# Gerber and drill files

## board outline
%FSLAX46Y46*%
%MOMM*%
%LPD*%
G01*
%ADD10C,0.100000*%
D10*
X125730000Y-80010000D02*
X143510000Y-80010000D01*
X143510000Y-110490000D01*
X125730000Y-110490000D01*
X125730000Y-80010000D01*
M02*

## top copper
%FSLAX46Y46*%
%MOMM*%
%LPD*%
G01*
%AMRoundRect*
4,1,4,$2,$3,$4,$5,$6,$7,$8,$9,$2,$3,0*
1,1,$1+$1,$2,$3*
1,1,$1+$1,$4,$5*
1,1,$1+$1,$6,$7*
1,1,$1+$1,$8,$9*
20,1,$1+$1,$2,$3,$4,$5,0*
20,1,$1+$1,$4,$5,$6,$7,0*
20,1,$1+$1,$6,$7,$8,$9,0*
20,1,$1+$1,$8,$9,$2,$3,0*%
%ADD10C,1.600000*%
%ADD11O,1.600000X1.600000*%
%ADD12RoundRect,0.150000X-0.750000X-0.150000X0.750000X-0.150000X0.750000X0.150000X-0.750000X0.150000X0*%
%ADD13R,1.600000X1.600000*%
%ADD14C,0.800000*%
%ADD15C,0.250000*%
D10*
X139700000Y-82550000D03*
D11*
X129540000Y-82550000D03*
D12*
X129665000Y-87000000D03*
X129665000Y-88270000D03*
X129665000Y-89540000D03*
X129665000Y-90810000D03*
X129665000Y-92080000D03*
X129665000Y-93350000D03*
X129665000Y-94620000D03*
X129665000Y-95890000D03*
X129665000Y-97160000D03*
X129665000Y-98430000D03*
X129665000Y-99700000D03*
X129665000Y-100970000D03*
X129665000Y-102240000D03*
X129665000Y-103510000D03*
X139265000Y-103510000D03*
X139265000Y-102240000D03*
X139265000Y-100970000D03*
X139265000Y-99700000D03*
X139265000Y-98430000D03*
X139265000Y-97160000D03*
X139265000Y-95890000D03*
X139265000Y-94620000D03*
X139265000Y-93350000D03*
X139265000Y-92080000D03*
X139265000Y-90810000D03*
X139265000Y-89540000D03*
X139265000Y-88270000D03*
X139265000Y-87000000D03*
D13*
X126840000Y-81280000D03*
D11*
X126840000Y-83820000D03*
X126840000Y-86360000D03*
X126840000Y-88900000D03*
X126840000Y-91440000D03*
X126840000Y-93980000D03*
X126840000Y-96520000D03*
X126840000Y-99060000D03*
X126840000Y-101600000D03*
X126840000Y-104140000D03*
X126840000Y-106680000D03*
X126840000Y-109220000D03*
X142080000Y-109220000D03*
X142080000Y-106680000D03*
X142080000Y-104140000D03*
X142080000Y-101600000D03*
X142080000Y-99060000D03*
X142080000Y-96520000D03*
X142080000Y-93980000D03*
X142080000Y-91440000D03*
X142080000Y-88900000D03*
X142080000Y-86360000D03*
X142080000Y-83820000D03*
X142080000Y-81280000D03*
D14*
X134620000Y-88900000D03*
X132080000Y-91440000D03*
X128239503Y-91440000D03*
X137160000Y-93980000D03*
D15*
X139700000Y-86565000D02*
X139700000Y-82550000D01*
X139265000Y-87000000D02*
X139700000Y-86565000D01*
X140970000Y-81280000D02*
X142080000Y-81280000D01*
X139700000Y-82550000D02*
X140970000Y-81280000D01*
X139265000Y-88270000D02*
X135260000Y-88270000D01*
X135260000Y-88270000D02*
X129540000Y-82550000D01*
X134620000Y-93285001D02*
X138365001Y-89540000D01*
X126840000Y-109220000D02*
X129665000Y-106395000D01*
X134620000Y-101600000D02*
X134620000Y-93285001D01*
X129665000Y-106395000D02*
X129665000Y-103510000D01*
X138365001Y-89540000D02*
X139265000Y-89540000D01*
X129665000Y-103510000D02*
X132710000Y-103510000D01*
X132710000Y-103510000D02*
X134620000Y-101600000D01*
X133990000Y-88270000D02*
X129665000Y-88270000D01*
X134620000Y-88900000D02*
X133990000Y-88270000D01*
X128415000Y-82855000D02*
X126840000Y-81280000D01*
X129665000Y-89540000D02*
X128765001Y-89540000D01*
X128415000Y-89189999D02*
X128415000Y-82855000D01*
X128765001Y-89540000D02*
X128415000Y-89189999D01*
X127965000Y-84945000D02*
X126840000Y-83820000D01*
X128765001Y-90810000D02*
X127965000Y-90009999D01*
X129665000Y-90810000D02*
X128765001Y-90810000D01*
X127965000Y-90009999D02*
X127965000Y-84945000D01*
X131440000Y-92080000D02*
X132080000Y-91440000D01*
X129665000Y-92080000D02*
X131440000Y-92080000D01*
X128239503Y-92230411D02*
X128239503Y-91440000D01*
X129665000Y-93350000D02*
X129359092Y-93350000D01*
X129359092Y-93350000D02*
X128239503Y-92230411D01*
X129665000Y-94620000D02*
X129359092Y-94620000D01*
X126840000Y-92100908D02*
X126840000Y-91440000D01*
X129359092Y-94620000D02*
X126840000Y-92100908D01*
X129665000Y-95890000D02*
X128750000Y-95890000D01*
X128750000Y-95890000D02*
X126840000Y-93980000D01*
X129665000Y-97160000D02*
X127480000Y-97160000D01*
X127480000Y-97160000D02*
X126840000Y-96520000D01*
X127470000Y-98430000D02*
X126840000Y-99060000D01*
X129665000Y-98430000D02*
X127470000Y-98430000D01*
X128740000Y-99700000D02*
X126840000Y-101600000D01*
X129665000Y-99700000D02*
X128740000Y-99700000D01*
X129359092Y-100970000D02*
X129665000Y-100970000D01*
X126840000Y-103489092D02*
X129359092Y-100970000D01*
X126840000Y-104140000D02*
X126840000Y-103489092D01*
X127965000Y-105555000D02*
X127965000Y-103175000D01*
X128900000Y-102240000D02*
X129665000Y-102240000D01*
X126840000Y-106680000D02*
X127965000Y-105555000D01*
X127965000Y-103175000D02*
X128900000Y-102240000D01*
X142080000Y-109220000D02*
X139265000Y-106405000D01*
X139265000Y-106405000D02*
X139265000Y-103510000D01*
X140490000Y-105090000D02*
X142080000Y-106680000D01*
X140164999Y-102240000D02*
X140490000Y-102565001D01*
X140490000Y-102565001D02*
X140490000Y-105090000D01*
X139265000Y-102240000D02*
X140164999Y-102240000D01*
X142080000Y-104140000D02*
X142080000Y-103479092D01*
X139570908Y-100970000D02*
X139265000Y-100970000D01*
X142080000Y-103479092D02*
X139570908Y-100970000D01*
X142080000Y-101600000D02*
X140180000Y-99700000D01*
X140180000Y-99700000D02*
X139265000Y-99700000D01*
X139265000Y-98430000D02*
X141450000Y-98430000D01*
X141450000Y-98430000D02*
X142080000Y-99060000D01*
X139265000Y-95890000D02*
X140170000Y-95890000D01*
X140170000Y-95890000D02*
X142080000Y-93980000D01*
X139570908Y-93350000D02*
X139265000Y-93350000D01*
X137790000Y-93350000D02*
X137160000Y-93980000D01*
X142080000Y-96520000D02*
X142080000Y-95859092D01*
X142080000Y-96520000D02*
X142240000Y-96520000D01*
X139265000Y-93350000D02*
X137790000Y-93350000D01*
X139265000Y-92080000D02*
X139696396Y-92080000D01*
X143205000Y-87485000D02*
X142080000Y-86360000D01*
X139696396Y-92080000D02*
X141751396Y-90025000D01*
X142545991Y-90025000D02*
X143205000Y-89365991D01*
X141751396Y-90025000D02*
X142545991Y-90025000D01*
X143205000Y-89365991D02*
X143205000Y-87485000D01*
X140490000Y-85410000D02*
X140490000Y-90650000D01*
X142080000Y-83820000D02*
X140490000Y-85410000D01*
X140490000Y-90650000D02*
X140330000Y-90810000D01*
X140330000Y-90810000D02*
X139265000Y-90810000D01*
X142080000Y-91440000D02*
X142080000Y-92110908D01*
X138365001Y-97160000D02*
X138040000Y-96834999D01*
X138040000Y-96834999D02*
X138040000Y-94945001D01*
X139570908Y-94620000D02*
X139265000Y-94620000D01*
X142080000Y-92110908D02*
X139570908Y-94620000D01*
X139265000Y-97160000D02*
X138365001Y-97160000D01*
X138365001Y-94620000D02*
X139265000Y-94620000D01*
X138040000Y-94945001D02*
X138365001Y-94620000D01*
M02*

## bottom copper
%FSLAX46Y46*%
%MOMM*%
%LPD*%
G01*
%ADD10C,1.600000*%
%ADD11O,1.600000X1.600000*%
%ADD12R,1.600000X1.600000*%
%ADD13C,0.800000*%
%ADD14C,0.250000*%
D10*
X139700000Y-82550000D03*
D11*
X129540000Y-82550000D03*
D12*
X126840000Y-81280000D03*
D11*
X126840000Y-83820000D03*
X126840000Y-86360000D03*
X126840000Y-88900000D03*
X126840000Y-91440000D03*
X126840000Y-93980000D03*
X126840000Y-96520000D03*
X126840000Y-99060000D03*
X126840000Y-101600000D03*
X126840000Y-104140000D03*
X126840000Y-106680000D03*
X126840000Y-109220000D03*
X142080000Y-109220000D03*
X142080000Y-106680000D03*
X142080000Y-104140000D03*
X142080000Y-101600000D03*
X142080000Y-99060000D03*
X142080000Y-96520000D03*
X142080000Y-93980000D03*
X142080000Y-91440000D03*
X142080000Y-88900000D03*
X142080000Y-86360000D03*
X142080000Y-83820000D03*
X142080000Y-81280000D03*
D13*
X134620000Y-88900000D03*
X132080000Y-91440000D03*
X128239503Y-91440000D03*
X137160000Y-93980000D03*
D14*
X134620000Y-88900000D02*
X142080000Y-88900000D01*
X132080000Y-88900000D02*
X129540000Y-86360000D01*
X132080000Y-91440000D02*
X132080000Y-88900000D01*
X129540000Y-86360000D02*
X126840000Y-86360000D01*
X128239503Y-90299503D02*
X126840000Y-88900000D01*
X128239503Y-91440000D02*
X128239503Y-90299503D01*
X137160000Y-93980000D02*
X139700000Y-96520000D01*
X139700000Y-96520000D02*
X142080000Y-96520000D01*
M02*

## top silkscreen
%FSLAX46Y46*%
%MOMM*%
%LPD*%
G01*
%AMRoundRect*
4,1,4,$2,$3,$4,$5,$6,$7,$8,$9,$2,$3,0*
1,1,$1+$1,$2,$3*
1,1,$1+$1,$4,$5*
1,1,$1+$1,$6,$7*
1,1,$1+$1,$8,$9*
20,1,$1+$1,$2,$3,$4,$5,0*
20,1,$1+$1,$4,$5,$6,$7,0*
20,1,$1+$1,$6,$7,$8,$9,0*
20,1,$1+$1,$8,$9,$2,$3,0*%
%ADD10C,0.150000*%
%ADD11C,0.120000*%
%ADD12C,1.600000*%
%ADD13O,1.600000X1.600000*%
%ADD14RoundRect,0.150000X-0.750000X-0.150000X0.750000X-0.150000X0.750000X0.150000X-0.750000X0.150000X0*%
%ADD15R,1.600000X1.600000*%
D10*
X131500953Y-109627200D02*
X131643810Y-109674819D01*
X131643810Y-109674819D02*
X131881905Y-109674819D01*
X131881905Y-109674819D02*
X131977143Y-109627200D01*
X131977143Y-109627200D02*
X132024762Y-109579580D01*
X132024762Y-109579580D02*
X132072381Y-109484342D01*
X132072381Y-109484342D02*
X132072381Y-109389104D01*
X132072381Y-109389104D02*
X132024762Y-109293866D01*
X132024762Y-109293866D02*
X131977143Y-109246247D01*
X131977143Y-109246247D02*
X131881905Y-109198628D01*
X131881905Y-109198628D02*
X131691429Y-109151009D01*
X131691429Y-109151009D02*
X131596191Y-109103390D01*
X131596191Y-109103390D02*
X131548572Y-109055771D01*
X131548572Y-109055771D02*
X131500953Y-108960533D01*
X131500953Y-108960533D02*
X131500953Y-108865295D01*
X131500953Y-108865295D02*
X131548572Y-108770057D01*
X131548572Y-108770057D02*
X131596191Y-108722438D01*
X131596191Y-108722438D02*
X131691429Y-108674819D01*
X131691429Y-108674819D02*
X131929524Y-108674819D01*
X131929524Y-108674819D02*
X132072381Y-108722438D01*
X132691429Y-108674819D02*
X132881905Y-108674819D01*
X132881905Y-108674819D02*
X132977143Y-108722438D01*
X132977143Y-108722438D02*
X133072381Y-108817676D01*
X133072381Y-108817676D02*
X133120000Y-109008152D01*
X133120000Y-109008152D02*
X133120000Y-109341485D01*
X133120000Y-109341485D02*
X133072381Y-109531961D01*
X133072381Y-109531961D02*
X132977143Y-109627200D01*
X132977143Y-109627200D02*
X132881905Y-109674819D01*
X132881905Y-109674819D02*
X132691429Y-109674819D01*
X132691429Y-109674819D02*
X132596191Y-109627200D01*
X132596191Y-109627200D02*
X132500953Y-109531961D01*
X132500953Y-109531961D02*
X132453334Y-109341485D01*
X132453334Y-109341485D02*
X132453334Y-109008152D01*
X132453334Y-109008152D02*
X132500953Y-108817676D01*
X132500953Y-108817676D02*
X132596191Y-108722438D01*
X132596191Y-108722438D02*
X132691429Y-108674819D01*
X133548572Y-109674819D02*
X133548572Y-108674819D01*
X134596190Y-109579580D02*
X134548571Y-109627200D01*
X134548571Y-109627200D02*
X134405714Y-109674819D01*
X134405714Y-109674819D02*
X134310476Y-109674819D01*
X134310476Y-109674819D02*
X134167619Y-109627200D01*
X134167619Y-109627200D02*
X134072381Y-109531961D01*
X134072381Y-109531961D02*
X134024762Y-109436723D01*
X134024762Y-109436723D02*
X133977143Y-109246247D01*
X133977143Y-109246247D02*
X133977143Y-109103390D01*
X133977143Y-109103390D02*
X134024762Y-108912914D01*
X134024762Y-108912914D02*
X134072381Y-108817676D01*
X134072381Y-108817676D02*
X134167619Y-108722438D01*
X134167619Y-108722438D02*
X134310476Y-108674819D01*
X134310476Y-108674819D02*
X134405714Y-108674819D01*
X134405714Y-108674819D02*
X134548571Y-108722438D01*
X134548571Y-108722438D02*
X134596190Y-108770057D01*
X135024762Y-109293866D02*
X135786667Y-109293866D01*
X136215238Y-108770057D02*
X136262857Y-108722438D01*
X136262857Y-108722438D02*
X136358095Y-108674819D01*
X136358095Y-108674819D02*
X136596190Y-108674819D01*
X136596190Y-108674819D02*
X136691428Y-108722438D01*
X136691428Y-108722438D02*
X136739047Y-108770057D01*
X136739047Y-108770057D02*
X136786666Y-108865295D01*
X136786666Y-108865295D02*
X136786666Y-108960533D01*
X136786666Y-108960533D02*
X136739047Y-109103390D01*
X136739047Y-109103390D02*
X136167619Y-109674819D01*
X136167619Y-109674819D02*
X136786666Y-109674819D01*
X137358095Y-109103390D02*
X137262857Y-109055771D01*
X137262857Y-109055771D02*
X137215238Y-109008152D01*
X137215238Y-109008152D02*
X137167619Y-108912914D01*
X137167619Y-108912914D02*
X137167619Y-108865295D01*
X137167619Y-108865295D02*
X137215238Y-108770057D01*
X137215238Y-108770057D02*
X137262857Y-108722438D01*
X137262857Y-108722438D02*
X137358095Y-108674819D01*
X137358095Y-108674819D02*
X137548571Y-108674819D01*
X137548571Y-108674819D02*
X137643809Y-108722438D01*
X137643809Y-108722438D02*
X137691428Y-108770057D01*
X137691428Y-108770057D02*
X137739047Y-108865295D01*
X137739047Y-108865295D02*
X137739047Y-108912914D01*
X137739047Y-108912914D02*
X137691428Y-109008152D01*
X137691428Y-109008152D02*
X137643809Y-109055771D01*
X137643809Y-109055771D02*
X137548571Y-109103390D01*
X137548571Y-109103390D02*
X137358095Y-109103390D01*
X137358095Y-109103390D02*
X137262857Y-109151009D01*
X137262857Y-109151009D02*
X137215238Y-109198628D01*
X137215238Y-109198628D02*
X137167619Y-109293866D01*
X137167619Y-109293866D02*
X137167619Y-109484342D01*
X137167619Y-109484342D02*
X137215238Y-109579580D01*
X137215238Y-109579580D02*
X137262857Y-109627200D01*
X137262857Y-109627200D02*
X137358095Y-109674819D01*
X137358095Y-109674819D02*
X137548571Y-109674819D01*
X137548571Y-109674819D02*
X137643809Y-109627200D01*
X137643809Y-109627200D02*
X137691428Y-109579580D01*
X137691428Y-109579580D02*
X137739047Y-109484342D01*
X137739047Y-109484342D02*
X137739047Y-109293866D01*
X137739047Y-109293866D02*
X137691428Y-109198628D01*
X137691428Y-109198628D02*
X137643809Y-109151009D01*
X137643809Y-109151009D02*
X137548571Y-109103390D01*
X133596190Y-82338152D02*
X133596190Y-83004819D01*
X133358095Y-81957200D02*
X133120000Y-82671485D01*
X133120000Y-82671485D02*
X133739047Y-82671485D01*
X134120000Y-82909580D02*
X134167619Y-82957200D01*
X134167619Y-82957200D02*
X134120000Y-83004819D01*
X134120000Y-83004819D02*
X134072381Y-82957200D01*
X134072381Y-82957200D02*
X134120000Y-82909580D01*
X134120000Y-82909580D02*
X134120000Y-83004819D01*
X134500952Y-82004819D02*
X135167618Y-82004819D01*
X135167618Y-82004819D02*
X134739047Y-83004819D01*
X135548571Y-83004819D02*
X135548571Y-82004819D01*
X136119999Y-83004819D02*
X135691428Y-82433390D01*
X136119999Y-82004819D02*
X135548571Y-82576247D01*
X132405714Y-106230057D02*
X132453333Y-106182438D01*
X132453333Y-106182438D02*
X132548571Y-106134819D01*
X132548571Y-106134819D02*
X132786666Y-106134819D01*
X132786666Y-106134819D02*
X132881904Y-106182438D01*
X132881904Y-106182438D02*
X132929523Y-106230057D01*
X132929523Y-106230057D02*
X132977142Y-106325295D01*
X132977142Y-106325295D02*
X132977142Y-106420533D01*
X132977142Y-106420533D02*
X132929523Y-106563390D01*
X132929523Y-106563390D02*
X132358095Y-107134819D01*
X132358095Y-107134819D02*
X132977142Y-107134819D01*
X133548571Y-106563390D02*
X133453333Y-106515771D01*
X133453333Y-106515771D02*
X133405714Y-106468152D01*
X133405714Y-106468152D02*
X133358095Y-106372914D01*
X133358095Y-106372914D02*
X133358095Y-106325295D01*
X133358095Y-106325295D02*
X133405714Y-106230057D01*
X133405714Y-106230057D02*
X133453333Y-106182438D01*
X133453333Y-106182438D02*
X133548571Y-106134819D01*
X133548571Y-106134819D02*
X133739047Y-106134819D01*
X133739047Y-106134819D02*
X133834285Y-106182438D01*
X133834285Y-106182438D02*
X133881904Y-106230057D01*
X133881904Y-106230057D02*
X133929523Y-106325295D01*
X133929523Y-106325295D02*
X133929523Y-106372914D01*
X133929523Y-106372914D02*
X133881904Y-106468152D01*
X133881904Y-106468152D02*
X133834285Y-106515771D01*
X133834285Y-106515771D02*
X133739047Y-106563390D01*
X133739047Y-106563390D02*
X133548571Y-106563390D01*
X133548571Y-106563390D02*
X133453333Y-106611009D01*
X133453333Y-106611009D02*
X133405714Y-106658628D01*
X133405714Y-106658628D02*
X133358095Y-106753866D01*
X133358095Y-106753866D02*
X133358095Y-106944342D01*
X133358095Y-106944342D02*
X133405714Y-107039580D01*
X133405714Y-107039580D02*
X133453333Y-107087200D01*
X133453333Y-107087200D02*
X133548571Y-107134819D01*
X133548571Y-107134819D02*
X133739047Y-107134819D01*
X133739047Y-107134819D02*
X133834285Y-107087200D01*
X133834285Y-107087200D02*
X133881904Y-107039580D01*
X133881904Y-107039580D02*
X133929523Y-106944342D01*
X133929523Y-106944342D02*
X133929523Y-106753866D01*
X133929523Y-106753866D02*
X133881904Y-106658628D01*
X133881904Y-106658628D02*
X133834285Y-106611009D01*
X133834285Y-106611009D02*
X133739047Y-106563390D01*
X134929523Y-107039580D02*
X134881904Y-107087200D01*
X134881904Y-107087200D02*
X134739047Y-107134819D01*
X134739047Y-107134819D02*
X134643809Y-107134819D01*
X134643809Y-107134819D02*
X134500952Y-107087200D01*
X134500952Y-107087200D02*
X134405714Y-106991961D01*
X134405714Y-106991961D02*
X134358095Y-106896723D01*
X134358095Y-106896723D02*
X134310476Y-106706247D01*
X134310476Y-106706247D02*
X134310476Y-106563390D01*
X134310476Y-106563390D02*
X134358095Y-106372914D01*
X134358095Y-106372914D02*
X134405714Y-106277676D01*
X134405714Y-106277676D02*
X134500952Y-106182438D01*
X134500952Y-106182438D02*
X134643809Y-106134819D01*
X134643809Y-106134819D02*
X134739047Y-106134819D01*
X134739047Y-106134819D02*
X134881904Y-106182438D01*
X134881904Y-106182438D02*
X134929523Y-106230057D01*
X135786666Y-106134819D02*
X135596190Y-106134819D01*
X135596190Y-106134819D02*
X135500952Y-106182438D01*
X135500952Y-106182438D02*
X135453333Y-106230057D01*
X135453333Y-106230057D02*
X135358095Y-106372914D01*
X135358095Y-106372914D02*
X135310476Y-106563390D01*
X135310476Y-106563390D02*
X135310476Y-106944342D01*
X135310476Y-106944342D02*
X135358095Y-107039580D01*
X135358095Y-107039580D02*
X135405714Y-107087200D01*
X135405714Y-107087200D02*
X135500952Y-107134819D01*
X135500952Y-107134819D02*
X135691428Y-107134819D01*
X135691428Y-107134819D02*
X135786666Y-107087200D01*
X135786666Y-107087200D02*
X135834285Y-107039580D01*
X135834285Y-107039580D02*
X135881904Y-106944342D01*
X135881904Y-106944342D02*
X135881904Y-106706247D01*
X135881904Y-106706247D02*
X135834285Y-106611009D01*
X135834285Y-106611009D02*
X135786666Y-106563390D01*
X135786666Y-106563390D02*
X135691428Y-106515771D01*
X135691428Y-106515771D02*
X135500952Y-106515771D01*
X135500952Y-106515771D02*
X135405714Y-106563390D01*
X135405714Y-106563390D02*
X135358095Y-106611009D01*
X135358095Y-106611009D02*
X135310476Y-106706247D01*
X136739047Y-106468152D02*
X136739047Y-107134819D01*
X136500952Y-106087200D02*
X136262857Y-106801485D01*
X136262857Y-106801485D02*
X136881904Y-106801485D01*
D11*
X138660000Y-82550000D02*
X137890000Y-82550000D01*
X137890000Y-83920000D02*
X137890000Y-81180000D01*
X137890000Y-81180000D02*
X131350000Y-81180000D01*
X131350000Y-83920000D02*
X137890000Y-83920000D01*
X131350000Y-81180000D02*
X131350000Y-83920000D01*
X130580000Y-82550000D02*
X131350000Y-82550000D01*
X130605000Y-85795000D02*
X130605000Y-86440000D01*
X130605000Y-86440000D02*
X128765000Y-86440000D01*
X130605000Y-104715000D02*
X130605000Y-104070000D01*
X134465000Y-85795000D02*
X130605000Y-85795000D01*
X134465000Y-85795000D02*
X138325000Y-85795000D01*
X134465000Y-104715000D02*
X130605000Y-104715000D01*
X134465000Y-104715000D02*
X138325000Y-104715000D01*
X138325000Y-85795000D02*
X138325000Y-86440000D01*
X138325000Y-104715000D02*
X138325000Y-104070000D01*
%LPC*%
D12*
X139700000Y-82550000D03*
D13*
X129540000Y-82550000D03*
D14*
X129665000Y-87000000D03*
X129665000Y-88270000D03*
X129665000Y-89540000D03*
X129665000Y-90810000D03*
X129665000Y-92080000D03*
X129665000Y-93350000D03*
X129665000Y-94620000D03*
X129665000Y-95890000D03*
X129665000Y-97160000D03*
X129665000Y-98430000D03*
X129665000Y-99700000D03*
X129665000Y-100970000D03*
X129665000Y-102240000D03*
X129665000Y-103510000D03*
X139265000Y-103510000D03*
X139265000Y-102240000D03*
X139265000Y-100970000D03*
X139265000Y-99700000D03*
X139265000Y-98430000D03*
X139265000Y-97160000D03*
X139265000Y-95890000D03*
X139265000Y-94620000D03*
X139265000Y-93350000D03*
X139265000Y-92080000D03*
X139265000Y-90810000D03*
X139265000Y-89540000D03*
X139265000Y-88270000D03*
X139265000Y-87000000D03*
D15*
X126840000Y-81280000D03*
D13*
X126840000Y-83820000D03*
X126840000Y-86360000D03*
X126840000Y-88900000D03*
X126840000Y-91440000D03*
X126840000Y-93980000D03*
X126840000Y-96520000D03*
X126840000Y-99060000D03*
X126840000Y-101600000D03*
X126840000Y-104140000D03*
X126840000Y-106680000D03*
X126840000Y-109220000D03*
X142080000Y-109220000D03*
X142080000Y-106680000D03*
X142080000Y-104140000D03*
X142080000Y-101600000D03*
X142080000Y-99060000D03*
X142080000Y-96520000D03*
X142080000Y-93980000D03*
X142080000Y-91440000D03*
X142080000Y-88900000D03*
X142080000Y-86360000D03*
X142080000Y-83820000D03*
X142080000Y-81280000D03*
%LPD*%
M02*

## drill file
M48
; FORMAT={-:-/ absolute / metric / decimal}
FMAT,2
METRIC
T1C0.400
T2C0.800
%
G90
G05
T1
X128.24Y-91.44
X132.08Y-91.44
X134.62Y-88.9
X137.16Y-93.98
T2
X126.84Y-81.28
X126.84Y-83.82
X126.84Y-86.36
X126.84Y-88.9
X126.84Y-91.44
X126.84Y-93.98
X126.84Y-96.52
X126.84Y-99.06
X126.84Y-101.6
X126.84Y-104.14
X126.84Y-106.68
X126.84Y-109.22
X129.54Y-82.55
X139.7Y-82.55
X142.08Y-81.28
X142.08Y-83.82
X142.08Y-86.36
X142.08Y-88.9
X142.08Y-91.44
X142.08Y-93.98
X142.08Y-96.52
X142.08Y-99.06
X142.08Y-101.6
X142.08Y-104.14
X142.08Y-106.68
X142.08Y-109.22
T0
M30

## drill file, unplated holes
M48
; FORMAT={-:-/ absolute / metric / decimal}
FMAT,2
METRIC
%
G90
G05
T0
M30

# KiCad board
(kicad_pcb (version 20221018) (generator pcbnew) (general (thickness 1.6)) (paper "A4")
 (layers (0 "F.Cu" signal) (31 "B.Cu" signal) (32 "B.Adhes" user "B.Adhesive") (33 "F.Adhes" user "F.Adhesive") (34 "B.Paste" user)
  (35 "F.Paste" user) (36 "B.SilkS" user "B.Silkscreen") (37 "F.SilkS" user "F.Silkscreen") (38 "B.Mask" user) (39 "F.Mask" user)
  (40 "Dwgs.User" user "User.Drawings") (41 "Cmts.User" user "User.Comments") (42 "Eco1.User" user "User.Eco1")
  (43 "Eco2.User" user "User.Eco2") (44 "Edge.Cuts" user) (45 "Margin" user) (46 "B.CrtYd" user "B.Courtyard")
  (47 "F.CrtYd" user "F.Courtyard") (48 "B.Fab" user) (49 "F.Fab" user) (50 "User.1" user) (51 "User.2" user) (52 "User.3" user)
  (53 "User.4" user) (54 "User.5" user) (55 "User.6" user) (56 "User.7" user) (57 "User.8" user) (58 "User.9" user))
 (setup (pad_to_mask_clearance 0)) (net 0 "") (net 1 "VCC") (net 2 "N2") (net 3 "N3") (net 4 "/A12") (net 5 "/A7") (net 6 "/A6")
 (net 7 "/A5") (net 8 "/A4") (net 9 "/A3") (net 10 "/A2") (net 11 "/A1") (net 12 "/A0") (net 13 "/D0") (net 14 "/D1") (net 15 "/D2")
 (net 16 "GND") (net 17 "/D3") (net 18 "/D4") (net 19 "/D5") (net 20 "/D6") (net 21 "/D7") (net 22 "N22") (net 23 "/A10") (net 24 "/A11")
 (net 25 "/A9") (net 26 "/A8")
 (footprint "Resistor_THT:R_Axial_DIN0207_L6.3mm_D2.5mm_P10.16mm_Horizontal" (layer "F.Cu") (at 139.7 82.55 180)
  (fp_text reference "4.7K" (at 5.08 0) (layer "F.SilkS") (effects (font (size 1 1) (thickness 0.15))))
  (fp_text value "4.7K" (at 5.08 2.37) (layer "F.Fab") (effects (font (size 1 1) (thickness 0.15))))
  (fp_line (start 1.04 0) (end 1.81 0) (stroke (width 0.12) (type solid)) (layer "F.SilkS"))
  (fp_line (start 1.81 -1.37) (end 1.81 1.37) (stroke (width 0.12) (type solid)) (layer "F.SilkS"))
  (fp_line (start 1.81 1.37) (end 8.35 1.37) (stroke (width 0.12) (type solid)) (layer "F.SilkS"))
  (fp_line (start 8.35 -1.37) (end 1.81 -1.37) (stroke (width 0.12) (type solid)) (layer "F.SilkS"))
  (fp_line (start 8.35 1.37) (end 8.35 -1.37) (stroke (width 0.12) (type solid)) (layer "F.SilkS"))
  (fp_line (start 9.12 0) (end 8.35 0) (stroke (width 0.12) (type solid)) (layer "F.SilkS"))
  (pad "1" thru_hole circle (at 0 0 180) (size 1.6 1.6) (drill 0.8) (layers "*.Cu" "*.Mask") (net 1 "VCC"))
  (pad "2" thru_hole oval (at 10.16 0 180) (size 1.6 1.6) (drill 0.8) (layers "*.Cu" "*.Mask") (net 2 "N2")))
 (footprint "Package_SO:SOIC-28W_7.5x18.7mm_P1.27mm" (layer "F.Cu") (at 134.465 95.255)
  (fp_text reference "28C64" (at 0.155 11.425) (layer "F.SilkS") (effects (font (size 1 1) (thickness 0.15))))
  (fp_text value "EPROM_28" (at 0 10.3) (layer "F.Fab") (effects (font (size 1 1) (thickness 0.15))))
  (fp_line (start -3.86 -9.46) (end -3.86 -8.815) (stroke (width 0.12) (type solid)) (layer "F.SilkS"))
  (fp_line (start -3.86 -8.815) (end -5.7 -8.815) (stroke (width 0.12) (type solid)) (layer "F.SilkS"))
  (fp_line (start -3.86 9.46) (end -3.86 8.815) (stroke (width 0.12) (type solid)) (layer "F.SilkS"))
  (fp_line (start 0 -9.46) (end -3.86 -9.46) (stroke (width 0.12) (type solid)) (layer "F.SilkS"))
  (fp_line (start 0 -9.46) (end 3.86 -9.46) (stroke (width 0.12) (type solid)) (layer "F.SilkS"))
  (fp_line (start 0 9.46) (end -3.86 9.46) (stroke (width 0.12) (type solid)) (layer "F.SilkS"))
  (fp_line (start 0 9.46) (end 3.86 9.46) (stroke (width 0.12) (type solid)) (layer "F.SilkS"))
  (fp_line (start 3.86 -9.46) (end 3.86 -8.815) (stroke (width 0.12) (type solid)) (layer "F.SilkS"))
  (fp_line (start 3.86 9.46) (end 3.86 8.815) (stroke (width 0.12) (type solid)) (layer "F.SilkS"))
  (pad "1" smd roundrect (at -4.8 -8.255) (size 1.8 0.6) (layers "F.Cu" "F.Paste" "F.Mask") (roundrect_rratio 0.25) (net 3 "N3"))
  (pad "2" smd roundrect (at -4.8 -6.985) (size 1.8 0.6) (layers "F.Cu" "F.Paste" "F.Mask") (roundrect_rratio 0.25) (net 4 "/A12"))
  (pad "3" smd roundrect (at -4.8 -5.715) (size 1.8 0.6) (layers "F.Cu" "F.Paste" "F.Mask") (roundrect_rratio 0.25) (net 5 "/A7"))
  (pad "4" smd roundrect (at -4.8 -4.445) (size 1.8 0.6) (layers "F.Cu" "F.Paste" "F.Mask") (roundrect_rratio 0.25) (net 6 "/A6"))
  (pad "5" smd roundrect (at -4.8 -3.175) (size 1.8 0.6) (layers "F.Cu" "F.Paste" "F.Mask") (roundrect_rratio 0.25) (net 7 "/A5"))
  (pad "6" smd roundrect (at -4.8 -1.905) (size 1.8 0.6) (layers "F.Cu" "F.Paste" "F.Mask") (roundrect_rratio 0.25) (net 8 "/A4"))
  (pad "7" smd roundrect (at -4.8 -0.635) (size 1.8 0.6) (layers "F.Cu" "F.Paste" "F.Mask") (roundrect_rratio 0.25) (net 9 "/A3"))
  (pad "8" smd roundrect (at -4.8 0.635) (size 1.8 0.6) (layers "F.Cu" "F.Paste" "F.Mask") (roundrect_rratio 0.25) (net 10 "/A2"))
  (pad "9" smd roundrect (at -4.8 1.905) (size 1.8 0.6) (layers "F.Cu" "F.Paste" "F.Mask") (roundrect_rratio 0.25) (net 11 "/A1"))
  (pad "10" smd roundrect (at -4.8 3.175) (size 1.8 0.6) (layers "F.Cu" "F.Paste" "F.Mask") (roundrect_rratio 0.25) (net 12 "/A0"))
  (pad "11" smd roundrect (at -4.8 4.445) (size 1.8 0.6) (layers "F.Cu" "F.Paste" "F.Mask") (roundrect_rratio 0.25) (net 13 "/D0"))
  (pad "12" smd roundrect (at -4.8 5.715) (size 1.8 0.6) (layers "F.Cu" "F.Paste" "F.Mask") (roundrect_rratio 0.25) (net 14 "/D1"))
  (pad "13" smd roundrect (at -4.8 6.985) (size 1.8 0.6) (layers "F.Cu" "F.Paste" "F.Mask") (roundrect_rratio 0.25) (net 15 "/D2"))
  (pad "14" smd roundrect (at -4.8 8.255) (size 1.8 0.6) (layers "F.Cu" "F.Paste" "F.Mask") (roundrect_rratio 0.25) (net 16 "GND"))
  (pad "15" smd roundrect (at 4.8 8.255) (size 1.8 0.6) (layers "F.Cu" "F.Paste" "F.Mask") (roundrect_rratio 0.25) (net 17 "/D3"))
  (pad "16" smd roundrect (at 4.8 6.985) (size 1.8 0.6) (layers "F.Cu" "F.Paste" "F.Mask") (roundrect_rratio 0.25) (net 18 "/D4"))
  (pad "17" smd roundrect (at 4.8 5.715) (size 1.8 0.6) (layers "F.Cu" "F.Paste" "F.Mask") (roundrect_rratio 0.25) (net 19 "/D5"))
  (pad "18" smd roundrect (at 4.8 4.445) (size 1.8 0.6) (layers "F.Cu" "F.Paste" "F.Mask") (roundrect_rratio 0.25) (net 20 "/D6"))
  (pad "19" smd roundrect (at 4.8 3.175) (size 1.8 0.6) (layers "F.Cu" "F.Paste" "F.Mask") (roundrect_rratio 0.25) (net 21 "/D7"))
  (pad "20" smd roundrect (at 4.8 1.905) (size 1.8 0.6) (layers "F.Cu" "F.Paste" "F.Mask") (roundrect_rratio 0.25) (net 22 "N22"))
  (pad "21" smd roundrect (at 4.8 0.635) (size 1.8 0.6) (layers "F.Cu" "F.Paste" "F.Mask") (roundrect_rratio 0.25) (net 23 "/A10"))
  (pad "22" smd roundrect (at 4.8 -0.635) (size 1.8 0.6) (layers "F.Cu" "F.Paste" "F.Mask") (roundrect_rratio 0.25) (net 22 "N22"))
  (pad "23" smd roundrect (at 4.8 -1.905) (size 1.8 0.6) (layers "F.Cu" "F.Paste" "F.Mask") (roundrect_rratio 0.25) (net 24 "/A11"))
  (pad "24" smd roundrect (at 4.8 -3.175) (size 1.8 0.6) (layers "F.Cu" "F.Paste" "F.Mask") (roundrect_rratio 0.25) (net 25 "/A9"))
  (pad "25" smd roundrect (at 4.8 -4.445) (size 1.8 0.6) (layers "F.Cu" "F.Paste" "F.Mask") (roundrect_rratio 0.25) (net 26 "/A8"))
  (pad "26" smd roundrect (at 4.8 -5.715) (size 1.8 0.6) (layers "F.Cu" "F.Paste" "F.Mask") (roundrect_rratio 0.25) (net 16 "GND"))
  (pad "27" smd roundrect (at 4.8 -6.985) (size 1.8 0.6) (layers "F.Cu" "F.Paste" "F.Mask") (roundrect_rratio 0.25) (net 2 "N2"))
  (pad "28" smd roundrect (at 4.8 -8.255) (size 1.8 0.6) (layers "F.Cu" "F.Paste" "F.Mask") (roundrect_rratio 0.25) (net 1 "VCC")))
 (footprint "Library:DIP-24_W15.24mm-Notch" (layer "F.Cu") (at 126.84 81.28)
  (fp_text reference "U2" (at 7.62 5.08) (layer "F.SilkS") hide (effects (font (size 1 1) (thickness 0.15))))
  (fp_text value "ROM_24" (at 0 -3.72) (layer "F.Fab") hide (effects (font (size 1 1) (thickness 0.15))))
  (pad "1" thru_hole rect (at 0 0) (size 1.6 1.6) (drill 0.8) (layers "*.Cu" "*.Mask") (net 5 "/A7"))
  (pad "2" thru_hole oval (at 0 2.54) (size 1.6 1.6) (drill 0.8) (layers "*.Cu" "*.Mask") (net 6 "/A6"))
  (pad "3" thru_hole oval (at 0 5.08) (size 1.6 1.6) (drill 0.8) (layers "*.Cu" "*.Mask") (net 7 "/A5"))
  (pad "4" thru_hole oval (at 0 7.62) (size 1.6 1.6) (drill 0.8) (layers "*.Cu" "*.Mask") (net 8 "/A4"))
  (pad "5" thru_hole oval (at 0 10.16) (size 1.6 1.6) (drill 0.8) (layers "*.Cu" "*.Mask") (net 9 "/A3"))
  (pad "6" thru_hole oval (at 0 12.7) (size 1.6 1.6) (drill 0.8) (layers "*.Cu" "*.Mask") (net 10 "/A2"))
  (pad "7" thru_hole oval (at 0 15.24) (size 1.6 1.6) (drill 0.8) (layers "*.Cu" "*.Mask") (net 11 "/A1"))
  (pad "8" thru_hole oval (at 0 17.78) (size 1.6 1.6) (drill 0.8) (layers "*.Cu" "*.Mask") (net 12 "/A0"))
  (pad "9" thru_hole oval (at 0 20.32) (size 1.6 1.6) (drill 0.8) (layers "*.Cu" "*.Mask") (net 13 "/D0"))
  (pad "10" thru_hole oval (at 0 22.86) (size 1.6 1.6) (drill 0.8) (layers "*.Cu" "*.Mask") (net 14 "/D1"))
  (pad "11" thru_hole oval (at 0 25.4) (size 1.6 1.6) (drill 0.8) (layers "*.Cu" "*.Mask") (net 15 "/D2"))
  (pad "12" thru_hole oval (at 0 27.94) (size 1.6 1.6) (drill 0.8) (layers "*.Cu" "*.Mask") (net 16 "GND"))
  (pad "13" thru_hole oval (at 15.24 27.94) (size 1.6 1.6) (drill 0.8) (layers "*.Cu" "*.Mask") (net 17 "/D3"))
  (pad "14" thru_hole oval (at 15.24 25.4) (size 1.6 1.6) (drill 0.8) (layers "*.Cu" "*.Mask") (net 18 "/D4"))
  (pad "15" thru_hole oval (at 15.24 22.86) (size 1.6 1.6) (drill 0.8) (layers "*.Cu" "*.Mask") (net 19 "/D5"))
  (pad "16" thru_hole oval (at 15.24 20.32) (size 1.6 1.6) (drill 0.8) (layers "*.Cu" "*.Mask") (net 20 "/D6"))
  (pad "17" thru_hole oval (at 15.24 17.78) (size 1.6 1.6) (drill 0.8) (layers "*.Cu" "*.Mask") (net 21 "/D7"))
  (pad "18" thru_hole oval (at 15.24 15.24) (size 1.6 1.6) (drill 0.8) (layers "*.Cu" "*.Mask") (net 24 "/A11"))
  (pad "19" thru_hole oval (at 15.24 12.7) (size 1.6 1.6) (drill 0.8) (layers "*.Cu" "*.Mask") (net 23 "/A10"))
  (pad "20" thru_hole oval (at 15.24 10.16) (size 1.6 1.6) (drill 0.8) (layers "*.Cu" "*.Mask") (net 22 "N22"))
  (pad "21" thru_hole oval (at 15.24 7.62) (size 1.6 1.6) (drill 0.8) (layers "*.Cu" "*.Mask") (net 4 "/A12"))
  (pad "22" thru_hole oval (at 15.24 5.08) (size 1.6 1.6) (drill 0.8) (layers "*.Cu" "*.Mask") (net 25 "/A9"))
  (pad "23" thru_hole oval (at 15.24 2.54) (size 1.6 1.6) (drill 0.8) (layers "*.Cu" "*.Mask") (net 26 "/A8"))
  (pad "24" thru_hole oval (at 15.24 0) (size 1.6 1.6) (drill 0.8) (layers "*.Cu" "*.Mask") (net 1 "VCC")))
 (gr_rect (start 125.73 80.01) (end 143.51 110.49) (stroke (width 0.1) (type default)) (fill none) (layer "Edge.Cuts"))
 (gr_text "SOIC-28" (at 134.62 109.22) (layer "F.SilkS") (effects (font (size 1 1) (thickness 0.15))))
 (segment (start 134.62 93.285001) (end 138.365001 89.54) (width 0.25) (layer "F.Cu") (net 16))
 (segment (start 126.84 109.22) (end 129.665 106.395) (width 0.25) (layer "F.Cu") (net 16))
 (segment (start 134.62 101.6) (end 134.62 93.285001) (width 0.25) (layer "F.Cu") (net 16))
 (segment (start 129.665 106.395) (end 129.665 103.51) (width 0.25) (layer "F.Cu") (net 16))
 (segment (start 138.365001 89.54) (end 139.265 89.54) (width 0.25) (layer "F.Cu") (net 16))
 (segment (start 129.665 103.51) (end 132.71 103.51) (width 0.25) (layer "F.Cu") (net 16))
 (segment (start 132.71 103.51) (end 134.62 101.6) (width 0.25) (layer "F.Cu") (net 16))
 (segment (start 133.99 88.27) (end 129.665 88.27) (width 0.25) (layer "F.Cu") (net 4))
 (segment (start 134.62 88.9) (end 133.99 88.27) (width 0.25) (layer "F.Cu") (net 4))
 (via (at 134.62 88.9) (size 0.8) (drill 0.4) (layers "F.Cu" "B.Cu") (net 4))
 (segment (start 134.62 88.9) (end 142.08 88.9) (width 0.25) (layer "B.Cu") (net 4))
 (segment (start 128.415 82.855) (end 126.84 81.28) (width 0.25) (layer "F.Cu") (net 5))
 (segment (start 129.665 89.54) (end 128.765001 89.54) (width 0.25) (layer "F.Cu") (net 5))
 (segment (start 128.415 89.189999) (end 128.415 82.855) (width 0.25) (layer "F.Cu") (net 5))
 (segment (start 128.765001 89.54) (end 128.415 89.189999) (width 0.25) (layer "F.Cu") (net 5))
 (segment (start 127.965 84.945) (end 126.84 83.82) (width 0.25) (layer "F.Cu") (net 6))
 (segment (start 128.765001 90.81) (end 127.965 90.009999) (width 0.25) (layer "F.Cu") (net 6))
 (segment (start 129.665 90.81) (end 128.765001 90.81) (width 0.25) (layer "F.Cu") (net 6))
 (segment (start 127.965 90.009999) (end 127.965 84.945) (width 0.25) (layer "F.Cu") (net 6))
 (segment (start 131.44 92.08) (end 132.08 91.44) (width 0.25) (layer "F.Cu") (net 7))
 (segment (start 129.665 92.08) (end 131.44 92.08) (width 0.25) (layer "F.Cu") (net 7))
 (via (at 132.08 91.44) (size 0.8) (drill 0.4) (layers "F.Cu" "B.Cu") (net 7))
 (segment (start 132.08 88.9) (end 129.54 86.36) (width 0.25) (layer "B.Cu") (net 7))
 (segment (start 132.08 91.44) (end 132.08 88.9) (width 0.25) (layer "B.Cu") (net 7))
 (segment (start 129.54 86.36) (end 126.84 86.36) (width 0.25) (layer "B.Cu") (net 7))
 (segment (start 128.239503 92.230411) (end 128.239503 91.44) (width 0.25) (layer "F.Cu") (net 8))
 (segment (start 129.665 93.35) (end 129.359092 93.35) (width 0.25) (layer "F.Cu") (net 8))
 (segment (start 129.359092 93.35) (end 128.239503 92.230411) (width 0.25) (layer "F.Cu") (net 8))
 (via (at 128.239503 91.44) (size 0.8) (drill 0.4) (layers "F.Cu" "B.Cu") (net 8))
 (segment (start 128.239503 90.299503) (end 126.84 88.9) (width 0.25) (layer "B.Cu") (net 8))
 (segment (start 128.239503 91.44) (end 128.239503 90.299503) (width 0.25) (layer "B.Cu") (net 8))
 (segment (start 129.665 94.62) (end 129.359092 94.62) (width 0.25) (layer "F.Cu") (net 9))
 (segment (start 126.84 92.100908) (end 126.84 91.44) (width 0.25) (layer "F.Cu") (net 9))
 (segment (start 129.359092 94.62) (end 126.84 92.100908) (width 0.25) (layer "F.Cu") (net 9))
 (segment (start 129.665 95.89) (end 128.75 95.89) (width 0.25) (layer "F.Cu") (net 10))
 (segment (start 128.75 95.89) (end 126.84 93.98) (width 0.25) (layer "F.Cu") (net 10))
 (segment (start 129.665 97.16) (end 127.48 97.16) (width 0.25) (layer "F.Cu") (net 11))
 (segment (start 127.48 97.16) (end 126.84 96.52) (width 0.25) (layer "F.Cu") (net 11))
 (segment (start 127.47 98.43) (end 126.84 99.06) (width 0.25) (layer "F.Cu") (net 12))
 (segment (start 129.665 98.43) (end 127.47 98.43) (width 0.25) (layer "F.Cu") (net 12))
 (segment (start 128.74 99.7) (end 126.84 101.6) (width 0.25) (layer "F.Cu") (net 13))
 (segment (start 129.665 99.7) (end 128.74 99.7) (width 0.25) (layer "F.Cu") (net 13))
 (segment (start 129.359092 100.97) (end 129.665 100.97) (width 0.25) (layer "F.Cu") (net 14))
 (segment (start 126.84 103.489092) (end 129.359092 100.97) (width 0.25) (layer "F.Cu") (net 14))
 (segment (start 126.84 104.14) (end 126.84 103.489092) (width 0.25) (layer "F.Cu") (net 14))
 (segment (start 127.965 105.555) (end 127.965 103.175) (width 0.25) (layer "F.Cu") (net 15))
 (segment (start 128.9 102.24) (end 129.665 102.24) (width 0.25) (layer "F.Cu") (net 15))
 (segment (start 126.84 106.68) (end 127.965 105.555) (width 0.25) (layer "F.Cu") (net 15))
 (segment (start 127.965 103.175) (end 128.9 102.24) (width 0.25) (layer "F.Cu") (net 15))
 (segment (start 142.08 109.22) (end 139.265 106.405) (width 0.25) (layer "F.Cu") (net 17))
 (segment (start 139.265 106.405) (end 139.265 103.51) (width 0.25) (layer "F.Cu") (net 17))
 (segment (start 140.49 105.09) (end 142.08 106.68) (width 0.25) (layer "F.Cu") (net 18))
 (segment (start 140.164999 102.24) (end 140.49 102.565001) (width 0.25) (layer "F.Cu") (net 18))
 (segment (start 140.49 102.565001) (end 140.49 105.09) (width 0.25) (layer "F.Cu") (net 18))
 (segment (start 139.265 102.24) (end 140.164999 102.24) (width 0.25) (layer "F.Cu") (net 18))
 (segment (start 142.08 104.14) (end 142.08 103.479092) (width 0.25) (layer "F.Cu") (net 19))
 (segment (start 139.570908 100.97) (end 139.265 100.97) (width 0.25) (layer "F.Cu") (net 19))
 (segment (start 142.08 103.479092) (end 139.570908 100.97) (width 0.25) (layer "F.Cu") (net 19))
 (segment (start 142.08 101.6) (end 140.18 99.7) (width 0.25) (layer "F.Cu") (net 20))
 (segment (start 140.18 99.7) (end 139.265 99.7) (width 0.25) (layer "F.Cu") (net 20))
 (segment (start 139.265 98.43) (end 141.45 98.43) (width 0.25) (layer "F.Cu") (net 21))
 (segment (start 141.45 98.43) (end 142.08 99.06) (width 0.25) (layer "F.Cu") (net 21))
 (segment (start 139.265 88.27) (end 135.26 88.27) (width 0.25) (layer "F.Cu") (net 2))
 (segment (start 135.26 88.27) (end 129.54 82.55) (width 0.25) (layer "F.Cu") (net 2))
 (segment (start 139.265 95.89) (end 140.17 95.89) (width 0.25) (layer "F.Cu") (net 23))
 (segment (start 140.17 95.89) (end 142.08 93.98) (width 0.25) (layer "F.Cu") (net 23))
 (segment (start 139.570908 93.35) (end 139.265 93.35) (width 0.25) (layer "F.Cu") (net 24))
 (segment (start 137.79 93.35) (end 137.16 93.98) (width 0.25) (layer "F.Cu") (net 24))
 (segment (start 142.08 96.52) (end 142.08 95.859092) (width 0.25) (layer "F.Cu") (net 24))
 (segment (start 142.08 96.52) (end 142.24 96.52) (width 0.25) (layer "F.Cu") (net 24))
 (segment (start 139.265 93.35) (end 137.79 93.35) (width 0.25) (layer "F.Cu") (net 24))
 (via (at 137.16 93.98) (size 0.8) (drill 0.4) (layers "F.Cu" "B.Cu") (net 24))
 (segment (start 137.16 93.98) (end 139.7 96.52) (width 0.25) (layer "B.Cu") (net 24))
 (segment (start 139.7 96.52) (end 142.08 96.52) (width 0.25) (layer "B.Cu") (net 24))
 (segment (start 139.265 92.08) (end 139.696396 92.08) (width 0.25) (layer "F.Cu") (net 25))
 (segment (start 143.205 87.485) (end 142.08 86.36) (width 0.25) (layer "F.Cu") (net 25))
 (segment (start 139.696396 92.08) (end 141.751396 90.025) (width 0.25) (layer "F.Cu") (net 25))
 (segment (start 142.545991 90.025) (end 143.205 89.365991) (width 0.25) (layer "F.Cu") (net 25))
 (segment (start 141.751396 90.025) (end 142.545991 90.025) (width 0.25) (layer "F.Cu") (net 25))
 (segment (start 143.205 89.365991) (end 143.205 87.485) (width 0.25) (layer "F.Cu") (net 25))
 (segment (start 140.49 85.41) (end 140.49 90.65) (width 0.25) (layer "F.Cu") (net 26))
 (segment (start 142.08 83.82) (end 140.49 85.41) (width 0.25) (layer "F.Cu") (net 26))
 (segment (start 140.49 90.65) (end 140.33 90.81) (width 0.25) (layer "F.Cu") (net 26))
 (segment (start 140.33 90.81) (end 139.265 90.81) (width 0.25) (layer "F.Cu") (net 26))
 (segment (start 139.7 82.55) (end 140.97 81.28) (width 0.25) (layer "F.Cu") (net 1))
 (segment (start 139.265 87) (end 139.7 86.565) (width 0.25) (layer "F.Cu") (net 1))
 (segment (start 140.97 81.28) (end 142.08 81.28) (width 0.25) (layer "F.Cu") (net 1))
 (segment (start 139.7 86.565) (end 139.7 82.55) (width 0.25) (layer "F.Cu") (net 1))
 (segment (start 142.08 91.44) (end 142.08 92.110908) (width 0.25) (layer "F.Cu") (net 22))
 (segment (start 138.365001 97.16) (end 138.04 96.834999) (width 0.25) (layer "F.Cu") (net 22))
 (segment (start 138.04 96.834999) (end 138.04 94.945001) (width 0.25) (layer "F.Cu") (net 22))
 (segment (start 139.570908 94.62) (end 139.265 94.62) (width 0.25) (layer "F.Cu") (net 22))
 (segment (start 142.08 92.110908) (end 139.570908 94.62) (width 0.25) (layer "F.Cu") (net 22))
 (segment (start 139.265 97.16) (end 138.365001 97.16) (width 0.25) (layer "F.Cu") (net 22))
 (segment (start 138.365001 94.62) (end 139.265 94.62) (width 0.25) (layer "F.Cu") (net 22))
 (segment (start 138.04 94.945001) (end 138.365001 94.62) (width 0.25) (layer "F.Cu") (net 22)))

